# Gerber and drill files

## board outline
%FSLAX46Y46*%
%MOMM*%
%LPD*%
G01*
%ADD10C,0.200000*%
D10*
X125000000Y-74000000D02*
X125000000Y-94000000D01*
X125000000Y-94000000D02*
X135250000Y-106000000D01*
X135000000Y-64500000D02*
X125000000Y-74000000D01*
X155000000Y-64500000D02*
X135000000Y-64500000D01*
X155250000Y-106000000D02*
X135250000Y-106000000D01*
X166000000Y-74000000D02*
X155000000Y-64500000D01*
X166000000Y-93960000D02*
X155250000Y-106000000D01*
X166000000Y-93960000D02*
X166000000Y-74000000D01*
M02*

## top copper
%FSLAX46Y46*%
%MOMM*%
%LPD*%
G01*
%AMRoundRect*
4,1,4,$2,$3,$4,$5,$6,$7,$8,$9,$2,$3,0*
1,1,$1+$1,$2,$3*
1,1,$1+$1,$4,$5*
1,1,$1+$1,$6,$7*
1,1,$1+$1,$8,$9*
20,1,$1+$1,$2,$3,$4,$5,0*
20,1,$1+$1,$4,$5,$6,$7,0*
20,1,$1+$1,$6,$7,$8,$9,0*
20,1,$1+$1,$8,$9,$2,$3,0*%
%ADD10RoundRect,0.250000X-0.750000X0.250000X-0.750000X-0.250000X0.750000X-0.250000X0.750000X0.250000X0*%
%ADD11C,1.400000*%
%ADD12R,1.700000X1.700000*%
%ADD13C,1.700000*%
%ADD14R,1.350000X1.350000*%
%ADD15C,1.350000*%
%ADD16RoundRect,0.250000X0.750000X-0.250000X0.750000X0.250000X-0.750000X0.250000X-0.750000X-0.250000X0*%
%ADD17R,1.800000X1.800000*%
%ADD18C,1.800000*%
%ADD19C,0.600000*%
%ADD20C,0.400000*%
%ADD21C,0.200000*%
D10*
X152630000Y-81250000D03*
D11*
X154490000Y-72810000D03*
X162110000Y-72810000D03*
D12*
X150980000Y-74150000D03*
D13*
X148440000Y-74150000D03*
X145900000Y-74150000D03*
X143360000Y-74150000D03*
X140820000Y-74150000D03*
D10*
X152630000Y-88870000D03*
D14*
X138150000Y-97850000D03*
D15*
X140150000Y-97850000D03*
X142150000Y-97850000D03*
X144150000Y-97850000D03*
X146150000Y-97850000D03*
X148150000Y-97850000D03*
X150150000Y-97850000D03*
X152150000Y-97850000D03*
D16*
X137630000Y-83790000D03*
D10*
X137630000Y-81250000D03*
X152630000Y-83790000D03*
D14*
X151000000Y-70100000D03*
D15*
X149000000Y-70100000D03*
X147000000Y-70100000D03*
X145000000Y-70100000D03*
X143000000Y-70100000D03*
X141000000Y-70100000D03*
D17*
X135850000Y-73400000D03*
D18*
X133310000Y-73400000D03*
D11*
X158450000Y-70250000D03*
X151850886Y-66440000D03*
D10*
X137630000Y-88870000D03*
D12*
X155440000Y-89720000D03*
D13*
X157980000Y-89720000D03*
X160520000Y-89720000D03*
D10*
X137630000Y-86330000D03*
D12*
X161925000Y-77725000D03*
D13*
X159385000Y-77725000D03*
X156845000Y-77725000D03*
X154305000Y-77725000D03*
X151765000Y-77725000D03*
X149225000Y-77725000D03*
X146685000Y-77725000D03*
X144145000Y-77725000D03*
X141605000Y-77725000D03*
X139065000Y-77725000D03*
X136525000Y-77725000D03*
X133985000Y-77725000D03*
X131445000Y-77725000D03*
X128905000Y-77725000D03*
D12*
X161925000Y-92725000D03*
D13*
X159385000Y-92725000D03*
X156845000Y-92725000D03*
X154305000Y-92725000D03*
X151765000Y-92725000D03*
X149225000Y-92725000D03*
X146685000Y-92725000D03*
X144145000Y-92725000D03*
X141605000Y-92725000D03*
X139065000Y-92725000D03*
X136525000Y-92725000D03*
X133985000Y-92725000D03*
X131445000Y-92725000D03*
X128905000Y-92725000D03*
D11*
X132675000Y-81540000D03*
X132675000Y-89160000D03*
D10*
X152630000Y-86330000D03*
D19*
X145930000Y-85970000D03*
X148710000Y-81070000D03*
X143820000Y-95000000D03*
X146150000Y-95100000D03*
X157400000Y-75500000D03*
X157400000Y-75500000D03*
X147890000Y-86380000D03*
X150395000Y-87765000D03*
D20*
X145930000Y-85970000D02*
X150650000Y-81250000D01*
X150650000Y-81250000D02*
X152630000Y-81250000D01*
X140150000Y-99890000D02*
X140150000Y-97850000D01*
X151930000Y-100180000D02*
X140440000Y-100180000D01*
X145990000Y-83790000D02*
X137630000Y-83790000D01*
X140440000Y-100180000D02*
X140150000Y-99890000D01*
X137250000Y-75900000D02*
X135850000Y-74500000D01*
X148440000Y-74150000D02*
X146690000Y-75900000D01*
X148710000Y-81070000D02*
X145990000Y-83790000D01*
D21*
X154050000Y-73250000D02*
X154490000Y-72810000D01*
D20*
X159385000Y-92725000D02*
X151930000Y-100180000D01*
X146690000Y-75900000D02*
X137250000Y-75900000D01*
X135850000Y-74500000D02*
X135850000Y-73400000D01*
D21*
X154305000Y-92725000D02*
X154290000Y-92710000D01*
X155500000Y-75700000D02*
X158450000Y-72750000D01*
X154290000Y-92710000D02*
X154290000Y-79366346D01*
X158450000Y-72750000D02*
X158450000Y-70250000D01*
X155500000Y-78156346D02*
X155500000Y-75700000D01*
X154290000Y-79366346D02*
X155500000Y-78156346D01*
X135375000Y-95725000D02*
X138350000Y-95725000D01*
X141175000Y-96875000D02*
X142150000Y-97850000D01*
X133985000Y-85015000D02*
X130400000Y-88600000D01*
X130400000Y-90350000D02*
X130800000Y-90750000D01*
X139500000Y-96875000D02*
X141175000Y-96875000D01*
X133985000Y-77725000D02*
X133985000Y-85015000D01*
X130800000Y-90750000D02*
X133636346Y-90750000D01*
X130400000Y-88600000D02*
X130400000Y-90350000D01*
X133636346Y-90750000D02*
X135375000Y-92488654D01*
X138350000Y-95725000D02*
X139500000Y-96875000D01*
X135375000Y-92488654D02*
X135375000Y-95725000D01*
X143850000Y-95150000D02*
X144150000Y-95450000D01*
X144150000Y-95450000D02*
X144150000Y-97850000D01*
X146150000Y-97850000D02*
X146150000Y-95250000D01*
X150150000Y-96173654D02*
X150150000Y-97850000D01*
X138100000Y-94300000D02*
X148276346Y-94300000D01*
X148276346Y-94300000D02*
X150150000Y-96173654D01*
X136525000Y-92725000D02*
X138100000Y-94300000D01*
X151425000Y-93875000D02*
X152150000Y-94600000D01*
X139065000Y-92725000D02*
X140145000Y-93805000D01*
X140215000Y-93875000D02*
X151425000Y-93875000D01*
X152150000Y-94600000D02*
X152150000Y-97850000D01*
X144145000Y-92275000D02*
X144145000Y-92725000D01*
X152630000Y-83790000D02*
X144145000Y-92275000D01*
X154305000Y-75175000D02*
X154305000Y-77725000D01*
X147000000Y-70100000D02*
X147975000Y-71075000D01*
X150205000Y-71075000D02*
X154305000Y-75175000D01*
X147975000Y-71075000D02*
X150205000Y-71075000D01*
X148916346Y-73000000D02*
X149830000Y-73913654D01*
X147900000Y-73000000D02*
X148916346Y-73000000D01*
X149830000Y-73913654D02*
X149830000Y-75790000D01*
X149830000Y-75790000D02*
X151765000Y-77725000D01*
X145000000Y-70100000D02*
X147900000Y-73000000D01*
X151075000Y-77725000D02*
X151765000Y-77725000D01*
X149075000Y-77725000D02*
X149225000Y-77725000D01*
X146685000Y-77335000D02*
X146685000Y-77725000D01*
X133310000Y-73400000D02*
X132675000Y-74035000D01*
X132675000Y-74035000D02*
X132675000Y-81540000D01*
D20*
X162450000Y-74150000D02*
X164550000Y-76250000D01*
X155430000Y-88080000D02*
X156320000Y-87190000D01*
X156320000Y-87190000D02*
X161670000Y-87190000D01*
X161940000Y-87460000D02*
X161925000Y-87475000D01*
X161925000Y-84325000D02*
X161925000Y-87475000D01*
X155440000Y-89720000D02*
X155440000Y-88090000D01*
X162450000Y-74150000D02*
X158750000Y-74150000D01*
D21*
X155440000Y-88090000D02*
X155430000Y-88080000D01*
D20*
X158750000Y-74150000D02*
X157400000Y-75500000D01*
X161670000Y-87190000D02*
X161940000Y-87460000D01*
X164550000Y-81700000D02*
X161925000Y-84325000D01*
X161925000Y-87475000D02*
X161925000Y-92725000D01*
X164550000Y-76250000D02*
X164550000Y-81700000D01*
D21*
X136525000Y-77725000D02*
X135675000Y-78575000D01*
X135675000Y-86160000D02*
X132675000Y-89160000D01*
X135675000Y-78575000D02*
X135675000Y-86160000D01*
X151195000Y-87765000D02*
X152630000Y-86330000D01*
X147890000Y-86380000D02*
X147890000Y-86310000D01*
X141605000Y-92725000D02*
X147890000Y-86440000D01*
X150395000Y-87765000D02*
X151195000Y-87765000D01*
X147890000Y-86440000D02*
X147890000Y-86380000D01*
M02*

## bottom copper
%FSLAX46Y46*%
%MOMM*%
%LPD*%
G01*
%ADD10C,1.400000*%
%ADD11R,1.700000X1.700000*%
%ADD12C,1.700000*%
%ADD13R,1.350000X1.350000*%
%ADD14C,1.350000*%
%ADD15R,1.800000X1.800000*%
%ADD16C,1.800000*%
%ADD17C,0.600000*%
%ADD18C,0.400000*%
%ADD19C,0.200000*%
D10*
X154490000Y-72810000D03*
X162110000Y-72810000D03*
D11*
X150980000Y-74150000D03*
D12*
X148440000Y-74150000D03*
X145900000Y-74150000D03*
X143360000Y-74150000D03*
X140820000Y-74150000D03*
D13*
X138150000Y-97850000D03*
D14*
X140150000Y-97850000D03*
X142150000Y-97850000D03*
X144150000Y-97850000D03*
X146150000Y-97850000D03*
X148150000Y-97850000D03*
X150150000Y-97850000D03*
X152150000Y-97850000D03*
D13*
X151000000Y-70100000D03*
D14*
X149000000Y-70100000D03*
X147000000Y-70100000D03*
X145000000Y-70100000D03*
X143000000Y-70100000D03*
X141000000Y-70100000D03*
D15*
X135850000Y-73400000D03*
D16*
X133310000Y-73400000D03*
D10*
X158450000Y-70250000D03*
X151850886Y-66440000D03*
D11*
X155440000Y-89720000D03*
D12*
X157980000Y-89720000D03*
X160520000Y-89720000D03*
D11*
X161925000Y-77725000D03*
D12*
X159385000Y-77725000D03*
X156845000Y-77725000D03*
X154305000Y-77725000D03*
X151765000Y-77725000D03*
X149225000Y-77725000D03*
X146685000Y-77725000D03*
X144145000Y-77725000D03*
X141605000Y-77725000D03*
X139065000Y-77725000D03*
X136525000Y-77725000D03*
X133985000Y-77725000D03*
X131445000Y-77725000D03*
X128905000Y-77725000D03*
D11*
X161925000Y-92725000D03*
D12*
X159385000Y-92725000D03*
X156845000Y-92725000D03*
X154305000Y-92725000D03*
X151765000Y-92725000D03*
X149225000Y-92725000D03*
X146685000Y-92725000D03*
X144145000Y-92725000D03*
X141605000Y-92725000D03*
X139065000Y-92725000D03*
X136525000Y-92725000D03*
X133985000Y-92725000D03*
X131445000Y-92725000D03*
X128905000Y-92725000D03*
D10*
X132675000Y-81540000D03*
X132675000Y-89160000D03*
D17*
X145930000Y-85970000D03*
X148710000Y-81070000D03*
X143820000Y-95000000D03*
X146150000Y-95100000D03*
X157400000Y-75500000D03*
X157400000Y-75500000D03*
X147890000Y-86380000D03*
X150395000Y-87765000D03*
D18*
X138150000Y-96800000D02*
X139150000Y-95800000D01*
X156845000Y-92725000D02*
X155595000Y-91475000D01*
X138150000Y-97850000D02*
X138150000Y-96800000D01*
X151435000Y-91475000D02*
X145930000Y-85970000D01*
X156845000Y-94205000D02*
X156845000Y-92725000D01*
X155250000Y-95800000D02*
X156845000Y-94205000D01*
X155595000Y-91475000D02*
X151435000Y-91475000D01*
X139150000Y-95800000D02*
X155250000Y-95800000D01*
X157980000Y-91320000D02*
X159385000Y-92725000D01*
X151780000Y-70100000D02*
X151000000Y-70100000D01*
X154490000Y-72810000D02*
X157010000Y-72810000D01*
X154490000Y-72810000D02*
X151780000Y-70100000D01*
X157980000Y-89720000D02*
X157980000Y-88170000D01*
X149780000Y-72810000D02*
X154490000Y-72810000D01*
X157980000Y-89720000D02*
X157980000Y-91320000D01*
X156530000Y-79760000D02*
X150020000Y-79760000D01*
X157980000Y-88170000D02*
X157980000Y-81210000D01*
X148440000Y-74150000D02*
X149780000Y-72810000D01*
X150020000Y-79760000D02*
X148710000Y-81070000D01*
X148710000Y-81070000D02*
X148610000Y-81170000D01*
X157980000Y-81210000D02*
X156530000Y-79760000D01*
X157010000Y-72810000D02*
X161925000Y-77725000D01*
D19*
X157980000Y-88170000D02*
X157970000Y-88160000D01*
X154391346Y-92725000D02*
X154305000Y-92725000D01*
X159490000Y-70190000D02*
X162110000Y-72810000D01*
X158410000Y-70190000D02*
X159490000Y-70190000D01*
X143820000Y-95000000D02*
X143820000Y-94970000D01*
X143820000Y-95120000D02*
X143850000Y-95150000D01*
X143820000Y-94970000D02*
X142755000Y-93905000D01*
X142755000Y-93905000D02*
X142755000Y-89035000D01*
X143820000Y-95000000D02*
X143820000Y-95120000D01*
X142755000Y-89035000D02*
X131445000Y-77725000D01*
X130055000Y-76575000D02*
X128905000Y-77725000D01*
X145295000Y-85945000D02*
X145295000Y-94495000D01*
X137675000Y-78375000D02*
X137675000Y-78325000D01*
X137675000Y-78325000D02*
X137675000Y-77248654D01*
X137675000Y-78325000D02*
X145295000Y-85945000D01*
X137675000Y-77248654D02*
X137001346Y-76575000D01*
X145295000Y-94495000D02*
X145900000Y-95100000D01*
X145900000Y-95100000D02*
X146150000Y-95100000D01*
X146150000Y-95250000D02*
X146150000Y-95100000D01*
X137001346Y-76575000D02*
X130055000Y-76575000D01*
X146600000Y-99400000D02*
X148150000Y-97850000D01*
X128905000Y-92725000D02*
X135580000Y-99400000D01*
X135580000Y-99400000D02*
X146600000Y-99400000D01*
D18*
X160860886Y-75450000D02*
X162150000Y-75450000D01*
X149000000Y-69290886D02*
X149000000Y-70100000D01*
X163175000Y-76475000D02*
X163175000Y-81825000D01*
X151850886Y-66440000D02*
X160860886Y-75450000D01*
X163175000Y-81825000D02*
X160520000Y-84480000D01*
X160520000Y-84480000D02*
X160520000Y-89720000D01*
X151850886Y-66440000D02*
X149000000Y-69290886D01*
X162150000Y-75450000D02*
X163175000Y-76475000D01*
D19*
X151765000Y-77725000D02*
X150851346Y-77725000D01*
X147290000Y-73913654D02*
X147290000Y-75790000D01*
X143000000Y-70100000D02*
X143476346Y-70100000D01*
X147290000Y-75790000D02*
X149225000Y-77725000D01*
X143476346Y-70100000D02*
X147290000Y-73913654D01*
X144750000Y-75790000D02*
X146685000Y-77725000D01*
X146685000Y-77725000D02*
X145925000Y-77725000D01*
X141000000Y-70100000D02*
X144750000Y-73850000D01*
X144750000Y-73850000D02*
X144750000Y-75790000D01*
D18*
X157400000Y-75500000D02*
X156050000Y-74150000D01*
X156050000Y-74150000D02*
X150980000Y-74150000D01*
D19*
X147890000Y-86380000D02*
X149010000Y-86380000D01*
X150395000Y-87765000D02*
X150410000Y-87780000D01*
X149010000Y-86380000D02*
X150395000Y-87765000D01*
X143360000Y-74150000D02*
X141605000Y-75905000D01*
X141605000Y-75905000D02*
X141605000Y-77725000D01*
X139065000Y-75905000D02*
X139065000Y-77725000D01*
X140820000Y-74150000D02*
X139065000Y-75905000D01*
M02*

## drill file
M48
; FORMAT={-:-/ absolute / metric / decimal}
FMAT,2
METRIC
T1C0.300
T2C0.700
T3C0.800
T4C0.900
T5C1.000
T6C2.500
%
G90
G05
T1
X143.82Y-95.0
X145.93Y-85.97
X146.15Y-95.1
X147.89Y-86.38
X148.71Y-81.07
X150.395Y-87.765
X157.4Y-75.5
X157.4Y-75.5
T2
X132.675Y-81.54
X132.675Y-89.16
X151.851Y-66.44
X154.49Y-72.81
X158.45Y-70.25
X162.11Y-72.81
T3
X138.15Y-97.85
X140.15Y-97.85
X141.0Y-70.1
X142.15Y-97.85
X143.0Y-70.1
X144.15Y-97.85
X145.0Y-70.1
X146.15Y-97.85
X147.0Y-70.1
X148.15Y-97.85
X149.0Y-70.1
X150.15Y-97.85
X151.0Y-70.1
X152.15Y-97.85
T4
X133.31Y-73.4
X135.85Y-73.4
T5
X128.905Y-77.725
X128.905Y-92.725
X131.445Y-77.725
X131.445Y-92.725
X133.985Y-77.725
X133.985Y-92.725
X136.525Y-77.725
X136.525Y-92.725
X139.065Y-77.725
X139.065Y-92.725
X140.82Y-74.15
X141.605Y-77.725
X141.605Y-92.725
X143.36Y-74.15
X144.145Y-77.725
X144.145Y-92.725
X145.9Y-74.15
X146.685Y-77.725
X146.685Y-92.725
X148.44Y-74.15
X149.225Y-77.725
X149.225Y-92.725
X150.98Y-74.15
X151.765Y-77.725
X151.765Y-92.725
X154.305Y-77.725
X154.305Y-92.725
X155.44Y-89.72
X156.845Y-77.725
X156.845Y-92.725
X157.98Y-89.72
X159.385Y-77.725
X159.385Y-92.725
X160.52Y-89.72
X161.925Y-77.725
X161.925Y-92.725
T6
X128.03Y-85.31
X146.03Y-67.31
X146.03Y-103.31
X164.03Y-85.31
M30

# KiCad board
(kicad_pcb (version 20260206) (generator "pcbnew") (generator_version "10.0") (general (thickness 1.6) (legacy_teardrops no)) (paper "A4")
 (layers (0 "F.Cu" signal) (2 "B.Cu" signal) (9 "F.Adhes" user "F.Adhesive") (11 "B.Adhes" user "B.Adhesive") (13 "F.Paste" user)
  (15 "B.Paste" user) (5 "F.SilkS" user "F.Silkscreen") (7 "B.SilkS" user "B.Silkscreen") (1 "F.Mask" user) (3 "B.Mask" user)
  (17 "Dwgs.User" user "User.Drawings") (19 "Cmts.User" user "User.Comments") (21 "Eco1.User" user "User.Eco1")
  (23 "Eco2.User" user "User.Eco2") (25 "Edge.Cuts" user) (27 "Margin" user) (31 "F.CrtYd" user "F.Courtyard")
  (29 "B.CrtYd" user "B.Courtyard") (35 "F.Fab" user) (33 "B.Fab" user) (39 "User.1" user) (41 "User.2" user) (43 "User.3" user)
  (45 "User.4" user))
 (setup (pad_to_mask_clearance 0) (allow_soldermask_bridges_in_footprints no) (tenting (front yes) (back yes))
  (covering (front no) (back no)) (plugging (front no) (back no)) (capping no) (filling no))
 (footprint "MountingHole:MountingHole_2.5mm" (layer "F.Cu") (at 154.997 70.924)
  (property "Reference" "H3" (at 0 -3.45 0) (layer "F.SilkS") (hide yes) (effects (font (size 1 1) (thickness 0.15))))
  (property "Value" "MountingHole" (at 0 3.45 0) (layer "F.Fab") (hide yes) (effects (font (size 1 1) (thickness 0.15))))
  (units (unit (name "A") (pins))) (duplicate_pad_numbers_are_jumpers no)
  (pad "" np_thru_hole circle (at 9.033 14.386) (size 2.5 2.5) (drill 2.5) (layers "*.Cu" "*.Mask")))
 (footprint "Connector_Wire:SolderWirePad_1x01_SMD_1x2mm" (layer "F.Cu") (at 152.63 81.25 -90)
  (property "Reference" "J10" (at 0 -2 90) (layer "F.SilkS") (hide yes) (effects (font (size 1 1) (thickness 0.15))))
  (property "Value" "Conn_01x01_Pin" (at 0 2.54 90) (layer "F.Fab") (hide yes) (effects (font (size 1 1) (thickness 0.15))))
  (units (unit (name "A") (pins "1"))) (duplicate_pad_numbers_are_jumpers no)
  (pad "1" smd roundrect (at 0 0 270) (size 1 2) (layers "F.Cu" "F.Mask") (roundrect_rratio 0.25) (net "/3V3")))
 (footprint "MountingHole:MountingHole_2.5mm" (layer "F.Cu") (at 126.93 68.71)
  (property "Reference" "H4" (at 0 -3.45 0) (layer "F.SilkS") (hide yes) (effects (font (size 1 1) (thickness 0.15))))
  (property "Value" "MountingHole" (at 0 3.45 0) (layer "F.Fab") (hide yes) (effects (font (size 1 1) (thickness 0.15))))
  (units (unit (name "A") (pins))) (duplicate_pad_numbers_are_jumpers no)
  (pad "" np_thru_hole circle (at 1.1 16.6) (size 2.5 2.5) (drill 2.5) (layers "*.Cu" "*.Mask")))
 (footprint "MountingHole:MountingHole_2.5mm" (layer "F.Cu") (at 147.106 84.455)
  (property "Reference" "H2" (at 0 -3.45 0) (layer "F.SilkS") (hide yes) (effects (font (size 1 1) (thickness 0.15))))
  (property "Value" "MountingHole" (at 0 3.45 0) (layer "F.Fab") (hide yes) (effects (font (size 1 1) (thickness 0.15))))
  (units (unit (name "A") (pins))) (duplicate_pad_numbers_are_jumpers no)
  (pad "" np_thru_hole circle (at -1.076 18.855) (size 2.5 2.5) (drill 2.5) (layers "*.Cu" "*.Mask")))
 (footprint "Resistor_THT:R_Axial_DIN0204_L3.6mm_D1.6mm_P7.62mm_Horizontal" (layer "F.Cu") (at 154.49 72.81)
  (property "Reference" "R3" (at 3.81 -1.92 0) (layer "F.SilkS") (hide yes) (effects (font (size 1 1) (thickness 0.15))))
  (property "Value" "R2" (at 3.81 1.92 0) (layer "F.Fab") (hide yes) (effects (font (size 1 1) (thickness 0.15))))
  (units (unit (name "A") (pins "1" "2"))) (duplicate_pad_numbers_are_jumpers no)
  (pad "1" thru_hole circle (at 0 0) (size 1.4 1.4) (drill 0.7) (layers "*.Cu" "*.Mask") (remove_unused_layers no) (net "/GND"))
  (pad "2" thru_hole circle (at 7.62 0) (size 1.4 1.4) (drill 0.7) (layers "*.Cu" "*.Mask") (remove_unused_layers no) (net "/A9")))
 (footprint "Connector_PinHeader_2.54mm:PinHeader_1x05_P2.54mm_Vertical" (layer "F.Cu") (at 150.98 74.15 -90)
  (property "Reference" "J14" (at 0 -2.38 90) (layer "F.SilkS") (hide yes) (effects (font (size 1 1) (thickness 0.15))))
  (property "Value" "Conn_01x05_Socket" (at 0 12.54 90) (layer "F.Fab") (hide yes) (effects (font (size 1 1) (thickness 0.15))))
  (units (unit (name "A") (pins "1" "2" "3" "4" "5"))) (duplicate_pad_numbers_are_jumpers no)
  (pad "1" thru_hole rect (at 0 0 270) (size 1.7 1.7) (drill 1) (layers "*.Cu" "*.Mask") (remove_unused_layers no) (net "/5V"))
  (pad "2" thru_hole circle (at 0 2.54 270) (size 1.7 1.7) (drill 1) (layers "*.Cu" "*.Mask") (remove_unused_layers no) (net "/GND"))
  (pad "3" thru_hole circle (at 0 5.08 270) (size 1.7 1.7) (drill 1) (layers "*.Cu" "*.Mask") (remove_unused_layers no)
   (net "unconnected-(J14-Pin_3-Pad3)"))
  (pad "4" thru_hole circle (at 0 7.62 270) (size 1.7 1.7) (drill 1) (layers "*.Cu" "*.Mask") (remove_unused_layers no) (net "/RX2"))
  (pad "5" thru_hole circle (at 0 10.16 270) (size 1.7 1.7) (drill 1) (layers "*.Cu" "*.Mask") (remove_unused_layers no) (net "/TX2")))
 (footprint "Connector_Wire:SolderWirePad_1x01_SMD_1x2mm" (layer "F.Cu") (at 152.63 88.87 -90)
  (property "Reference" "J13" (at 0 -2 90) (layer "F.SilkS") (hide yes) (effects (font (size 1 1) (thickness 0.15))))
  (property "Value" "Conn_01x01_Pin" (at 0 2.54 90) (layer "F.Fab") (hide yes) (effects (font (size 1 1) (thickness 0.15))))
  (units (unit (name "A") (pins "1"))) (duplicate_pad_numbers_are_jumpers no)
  (pad "1" smd roundrect (at 0 0 270) (size 1 2) (layers "F.Cu" "F.Mask") (roundrect_rratio 0.25) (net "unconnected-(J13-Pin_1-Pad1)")))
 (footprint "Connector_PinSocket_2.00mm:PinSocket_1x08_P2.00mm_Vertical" (layer "F.Cu") (at 138.15 97.85 90)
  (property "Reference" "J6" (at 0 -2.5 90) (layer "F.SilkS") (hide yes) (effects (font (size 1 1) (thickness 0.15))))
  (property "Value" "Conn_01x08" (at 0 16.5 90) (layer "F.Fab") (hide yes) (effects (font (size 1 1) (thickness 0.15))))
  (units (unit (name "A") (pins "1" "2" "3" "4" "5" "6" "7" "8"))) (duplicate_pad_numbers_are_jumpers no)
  (pad "1" thru_hole rect (at 0 0 90) (size 1.35 1.35) (drill 0.8) (layers "*.Cu" "*.Mask") (remove_unused_layers no) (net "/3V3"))
  (pad "2" thru_hole circle (at 0 2 90) (size 1.35 1.35) (drill 0.8) (layers "*.Cu" "*.Mask") (remove_unused_layers no) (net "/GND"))
  (pad "3" thru_hole circle (at 0 4 90) (size 1.35 1.35) (drill 0.8) (layers "*.Cu" "*.Mask") (remove_unused_layers no) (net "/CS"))
  (pad "4" thru_hole circle (at 0 6 90) (size 1.35 1.35) (drill 0.8) (layers "*.Cu" "*.Mask") (remove_unused_layers no) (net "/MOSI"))
  (pad "5" thru_hole circle (at 0 8 90) (size 1.35 1.35) (drill 0.8) (layers "*.Cu" "*.Mask") (remove_unused_layers no) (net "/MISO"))
  (pad "6" thru_hole circle (at 0 10 90) (size 1.35 1.35) (drill 0.8) (layers "*.Cu" "*.Mask") (remove_unused_layers no) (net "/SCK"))
  (pad "7" thru_hole circle (at 0 12 90) (size 1.35 1.35) (drill 0.8) (layers "*.Cu" "*.Mask") (remove_unused_layers no) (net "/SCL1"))
  (pad "8" thru_hole circle (at 0 14 90) (size 1.35 1.35) (drill 0.8) (layers "*.Cu" "*.Mask") (remove_unused_layers no) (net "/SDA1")))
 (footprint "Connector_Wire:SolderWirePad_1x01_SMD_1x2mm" (layer "F.Cu") (at 137.63 83.79 90)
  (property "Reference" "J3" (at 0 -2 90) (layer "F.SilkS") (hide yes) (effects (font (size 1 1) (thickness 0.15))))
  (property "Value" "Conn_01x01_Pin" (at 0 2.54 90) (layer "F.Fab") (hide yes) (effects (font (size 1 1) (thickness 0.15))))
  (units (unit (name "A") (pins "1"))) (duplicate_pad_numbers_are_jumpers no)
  (pad "1" smd roundrect (at 0 0 90) (size 1 2) (layers "F.Cu" "F.Mask") (roundrect_rratio 0.25) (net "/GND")))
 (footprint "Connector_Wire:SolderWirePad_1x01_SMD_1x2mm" (layer "F.Cu") (at 137.63 81.25 -90)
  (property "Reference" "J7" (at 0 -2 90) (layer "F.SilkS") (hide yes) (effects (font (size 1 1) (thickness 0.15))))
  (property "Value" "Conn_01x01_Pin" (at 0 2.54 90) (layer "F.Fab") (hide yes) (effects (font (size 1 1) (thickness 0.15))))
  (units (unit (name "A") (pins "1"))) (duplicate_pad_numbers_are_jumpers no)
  (pad "1" smd roundrect (at 0 0 270) (size 1 2) (layers "F.Cu" "F.Mask") (roundrect_rratio 0.25) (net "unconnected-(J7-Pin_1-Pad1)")))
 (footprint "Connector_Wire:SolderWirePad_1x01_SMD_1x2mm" (layer "F.Cu") (at 152.63 83.79 -90)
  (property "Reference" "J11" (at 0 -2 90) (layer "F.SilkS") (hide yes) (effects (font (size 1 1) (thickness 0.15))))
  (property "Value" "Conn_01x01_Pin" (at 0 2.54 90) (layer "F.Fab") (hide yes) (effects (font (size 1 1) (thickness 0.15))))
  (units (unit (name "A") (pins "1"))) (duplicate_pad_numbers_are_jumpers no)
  (pad "1" smd roundrect (at 0 0 270) (size 1 2) (layers "F.Cu" "F.Mask") (roundrect_rratio 0.25) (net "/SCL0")))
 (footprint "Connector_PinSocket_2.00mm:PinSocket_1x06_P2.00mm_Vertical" (layer "F.Cu") (at 151 70.1 -90)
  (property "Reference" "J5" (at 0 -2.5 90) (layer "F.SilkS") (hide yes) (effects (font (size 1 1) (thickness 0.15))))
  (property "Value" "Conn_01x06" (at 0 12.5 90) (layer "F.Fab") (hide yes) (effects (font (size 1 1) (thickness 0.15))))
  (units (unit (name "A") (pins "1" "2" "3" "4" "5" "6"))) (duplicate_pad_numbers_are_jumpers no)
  (pad "1" thru_hole rect (at 0 0 270) (size 1.35 1.35) (drill 0.8) (layers "*.Cu" "*.Mask") (remove_unused_layers no) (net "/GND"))
  (pad "2" thru_hole circle (at 0 2 270) (size 1.35 1.35) (drill 0.8) (layers "*.Cu" "*.Mask") (remove_unused_layers no) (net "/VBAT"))
  (pad "3" thru_hole circle (at 0 4 270) (size 1.35 1.35) (drill 0.8) (layers "*.Cu" "*.Mask") (remove_unused_layers no) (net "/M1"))
  (pad "4" thru_hole circle (at 0 6 270) (size 1.35 1.35) (drill 0.8) (layers "*.Cu" "*.Mask") (remove_unused_layers no) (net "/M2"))
  (pad "5" thru_hole circle (at 0 8 270) (size 1.35 1.35) (drill 0.8) (layers "*.Cu" "*.Mask") (remove_unused_layers no) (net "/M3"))
  (pad "6" thru_hole circle (at 0 10 270) (size 1.35 1.35) (drill 0.8) (layers "*.Cu" "*.Mask") (remove_unused_layers no) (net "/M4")))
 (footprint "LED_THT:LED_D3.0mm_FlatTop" (layer "F.Cu") (at 135.85 73.4 180)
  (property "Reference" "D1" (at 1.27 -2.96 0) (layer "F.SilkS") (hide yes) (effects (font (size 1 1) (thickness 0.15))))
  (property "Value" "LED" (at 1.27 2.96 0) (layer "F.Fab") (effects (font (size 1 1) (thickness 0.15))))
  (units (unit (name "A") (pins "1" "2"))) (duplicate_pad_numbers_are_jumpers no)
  (pad "1" thru_hole rect (at 0 0 180) (size 1.8 1.8) (drill 0.9) (layers "*.Cu" "*.Mask") (remove_unused_layers no) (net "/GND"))
  (pad "2" thru_hole circle (at 2.54 0 180) (size 1.8 1.8) (drill 0.9) (layers "*.Cu" "*.Mask") (remove_unused_layers no) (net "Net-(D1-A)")))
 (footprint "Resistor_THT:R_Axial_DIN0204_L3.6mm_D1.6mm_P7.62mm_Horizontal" (layer "F.Cu") (at 158.45 70.25 150)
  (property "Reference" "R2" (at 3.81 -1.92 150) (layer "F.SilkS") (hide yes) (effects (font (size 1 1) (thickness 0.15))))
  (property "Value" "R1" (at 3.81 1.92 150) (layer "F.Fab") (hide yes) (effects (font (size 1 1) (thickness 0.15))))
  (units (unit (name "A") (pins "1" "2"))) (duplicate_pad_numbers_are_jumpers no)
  (pad "1" thru_hole circle (at 0 0 150) (size 1.4 1.4) (drill 0.7) (layers "*.Cu" "*.Mask") (remove_unused_layers no) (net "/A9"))
  (pad "2" thru_hole circle (at 7.62 0 150) (size 1.4 1.4) (drill 0.7) (layers "*.Cu" "*.Mask") (remove_unused_layers no) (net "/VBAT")))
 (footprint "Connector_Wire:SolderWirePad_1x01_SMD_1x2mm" (layer "F.Cu") (at 137.63 88.87 -90)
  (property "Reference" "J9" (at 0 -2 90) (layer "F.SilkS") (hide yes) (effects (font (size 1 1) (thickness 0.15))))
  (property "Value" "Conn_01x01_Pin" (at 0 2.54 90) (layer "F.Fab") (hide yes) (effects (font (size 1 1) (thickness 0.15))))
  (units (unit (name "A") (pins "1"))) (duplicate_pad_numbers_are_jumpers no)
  (pad "1" smd roundrect (at 0 0 270) (size 1 2) (layers "F.Cu" "F.Mask") (roundrect_rratio 0.25) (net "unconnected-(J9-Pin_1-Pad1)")))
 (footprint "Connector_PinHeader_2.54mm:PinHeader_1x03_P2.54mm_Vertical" (layer "F.Cu") (at 155.44 89.72 90)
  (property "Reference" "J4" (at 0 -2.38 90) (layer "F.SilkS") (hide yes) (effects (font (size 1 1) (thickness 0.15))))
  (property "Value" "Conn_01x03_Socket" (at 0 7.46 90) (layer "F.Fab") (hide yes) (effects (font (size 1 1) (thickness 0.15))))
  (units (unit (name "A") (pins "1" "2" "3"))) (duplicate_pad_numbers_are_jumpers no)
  (pad "1" thru_hole rect (at 0 0 90) (size 1.7 1.7) (drill 1) (layers "*.Cu" "*.Mask") (remove_unused_layers no) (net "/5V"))
  (pad "2" thru_hole circle (at 0 2.54 90) (size 1.7 1.7) (drill 1) (layers "*.Cu" "*.Mask") (remove_unused_layers no) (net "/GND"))
  (pad "3" thru_hole circle (at 0 5.08 90) (size 1.7 1.7) (drill 1) (layers "*.Cu" "*.Mask") (remove_unused_layers no) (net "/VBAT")))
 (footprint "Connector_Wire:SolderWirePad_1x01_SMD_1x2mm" (layer "F.Cu") (at 137.63 86.33 -90)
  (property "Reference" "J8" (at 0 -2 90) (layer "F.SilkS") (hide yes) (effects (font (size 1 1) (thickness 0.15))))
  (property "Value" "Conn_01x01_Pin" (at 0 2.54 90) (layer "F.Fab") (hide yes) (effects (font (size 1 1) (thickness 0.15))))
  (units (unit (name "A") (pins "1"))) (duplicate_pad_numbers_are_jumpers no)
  (pad "1" smd roundrect (at 0 0 270) (size 1 2) (layers "F.Cu" "F.Mask") (roundrect_rratio 0.25) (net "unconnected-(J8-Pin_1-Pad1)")))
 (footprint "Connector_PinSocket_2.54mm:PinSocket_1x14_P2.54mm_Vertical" (layer "F.Cu") (at 161.925 77.725 -90)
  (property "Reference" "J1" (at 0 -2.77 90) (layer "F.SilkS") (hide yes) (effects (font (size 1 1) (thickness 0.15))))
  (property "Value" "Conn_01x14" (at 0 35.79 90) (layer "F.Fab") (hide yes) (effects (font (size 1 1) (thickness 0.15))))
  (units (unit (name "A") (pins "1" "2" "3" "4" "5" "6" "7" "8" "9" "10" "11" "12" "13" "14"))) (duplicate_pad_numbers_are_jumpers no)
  (pad "1" thru_hole rect (at 0 0 270) (size 1.7 1.7) (drill 1) (layers "*.Cu" "*.Mask") (remove_unused_layers no) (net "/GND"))
  (pad "2" thru_hole circle (at 0 2.54 270) (size 1.7 1.7) (drill 1) (layers "*.Cu" "*.Mask") (remove_unused_layers no) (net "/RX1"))
  (pad "3" thru_hole circle (at 0 5.08 270) (size 1.7 1.7) (drill 1) (layers "*.Cu" "*.Mask") (remove_unused_layers no) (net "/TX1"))
  (pad "4" thru_hole circle (at 0 7.62 270) (size 1.7 1.7) (drill 1) (layers "*.Cu" "*.Mask") (remove_unused_layers no) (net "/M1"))
  (pad "5" thru_hole circle (at 0 10.16 270) (size 1.7 1.7) (drill 1) (layers "*.Cu" "*.Mask") (remove_unused_layers no) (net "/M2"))
  (pad "6" thru_hole circle (at 0 12.7 270) (size 1.7 1.7) (drill 1) (layers "*.Cu" "*.Mask") (remove_unused_layers no) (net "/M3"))
  (pad "7" thru_hole circle (at 0 15.24 270) (size 1.7 1.7) (drill 1) (layers "*.Cu" "*.Mask") (remove_unused_layers no) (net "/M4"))
  (pad "8" thru_hole circle (at 0 17.78 270) (size 1.7 1.7) (drill 1) (layers "*.Cu" "*.Mask") (remove_unused_layers no)
   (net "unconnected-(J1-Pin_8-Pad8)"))
  (pad "9" thru_hole circle (at 0 20.32 270) (size 1.7 1.7) (drill 1) (layers "*.Cu" "*.Mask") (remove_unused_layers no) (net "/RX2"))
  (pad "10" thru_hole circle (at 0 22.86 270) (size 1.7 1.7) (drill 1) (layers "*.Cu" "*.Mask") (remove_unused_layers no) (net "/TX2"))
  (pad "11" thru_hole circle (at 0 25.4 270) (size 1.7 1.7) (drill 1) (layers "*.Cu" "*.Mask") (remove_unused_layers no) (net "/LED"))
  (pad "12" thru_hole circle (at 0 27.94 270) (size 1.7 1.7) (drill 1) (layers "*.Cu" "*.Mask") (remove_unused_layers no) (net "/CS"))
  (pad "13" thru_hole circle (at 0 30.48 270) (size 1.7 1.7) (drill 1) (layers "*.Cu" "*.Mask") (remove_unused_layers no) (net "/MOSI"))
  (pad "14" thru_hole circle (at 0 33.02 270) (size 1.7 1.7) (drill 1) (layers "*.Cu" "*.Mask") (remove_unused_layers no) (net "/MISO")))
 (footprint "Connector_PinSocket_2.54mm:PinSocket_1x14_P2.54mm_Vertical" (layer "F.Cu") (at 161.925 92.725 -90)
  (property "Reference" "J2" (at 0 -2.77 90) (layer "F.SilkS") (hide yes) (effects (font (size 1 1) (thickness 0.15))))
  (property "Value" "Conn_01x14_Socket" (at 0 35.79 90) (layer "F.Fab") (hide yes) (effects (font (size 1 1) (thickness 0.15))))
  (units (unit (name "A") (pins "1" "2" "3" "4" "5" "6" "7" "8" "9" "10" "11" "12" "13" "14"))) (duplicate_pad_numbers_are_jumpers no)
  (pad "1" thru_hole rect (at 0 0 270) (size 1.7 1.7) (drill 1) (layers "*.Cu" "*.Mask") (remove_unused_layers no) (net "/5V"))
  (pad "2" thru_hole circle (at 0 2.54 270) (size 1.7 1.7) (drill 1) (layers "*.Cu" "*.Mask") (remove_unused_layers no) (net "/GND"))
  (pad "3" thru_hole circle (at 0 5.08 270) (size 1.7 1.7) (drill 1) (layers "*.Cu" "*.Mask") (remove_unused_layers no) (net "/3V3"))
  (pad "4" thru_hole circle (at 0 7.62 270) (size 1.7 1.7) (drill 1) (layers "*.Cu" "*.Mask") (remove_unused_layers no) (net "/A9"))
  (pad "5" thru_hole circle (at 0 10.16 270) (size 1.7 1.7) (drill 1) (layers "*.Cu" "*.Mask") (remove_unused_layers no)
   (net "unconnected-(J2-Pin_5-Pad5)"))
  (pad "6" thru_hole circle (at 0 12.7 270) (size 1.7 1.7) (drill 1) (layers "*.Cu" "*.Mask") (remove_unused_layers no)
   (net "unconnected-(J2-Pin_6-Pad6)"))
  (pad "7" thru_hole circle (at 0 15.24 270) (size 1.7 1.7) (drill 1) (layers "*.Cu" "*.Mask") (remove_unused_layers no)
   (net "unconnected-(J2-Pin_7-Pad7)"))
  (pad "8" thru_hole circle (at 0 17.78 270) (size 1.7 1.7) (drill 1) (layers "*.Cu" "*.Mask") (remove_unused_layers no) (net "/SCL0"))
  (pad "9" thru_hole circle (at 0 20.32 270) (size 1.7 1.7) (drill 1) (layers "*.Cu" "*.Mask") (remove_unused_layers no) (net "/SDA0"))
  (pad "10" thru_hole circle (at 0 22.86 270) (size 1.7 1.7) (drill 1) (layers "*.Cu" "*.Mask") (remove_unused_layers no) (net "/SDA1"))
  (pad "11" thru_hole circle (at 0 25.4 270) (size 1.7 1.7) (drill 1) (layers "*.Cu" "*.Mask") (remove_unused_layers no) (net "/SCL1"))
  (pad "12" thru_hole circle (at 0 27.94 270) (size 1.7 1.7) (drill 1) (layers "*.Cu" "*.Mask") (remove_unused_layers no) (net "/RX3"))
  (pad "13" thru_hole circle (at 0 30.48 270) (size 1.7 1.7) (drill 1) (layers "*.Cu" "*.Mask") (remove_unused_layers no) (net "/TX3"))
  (pad "14" thru_hole circle (at 0 33.02 270) (size 1.7 1.7) (drill 1) (layers "*.Cu" "*.Mask") (remove_unused_layers no) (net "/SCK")))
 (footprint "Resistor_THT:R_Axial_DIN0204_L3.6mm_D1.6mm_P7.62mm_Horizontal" (layer "F.Cu") (at 132.675 82.79 -90)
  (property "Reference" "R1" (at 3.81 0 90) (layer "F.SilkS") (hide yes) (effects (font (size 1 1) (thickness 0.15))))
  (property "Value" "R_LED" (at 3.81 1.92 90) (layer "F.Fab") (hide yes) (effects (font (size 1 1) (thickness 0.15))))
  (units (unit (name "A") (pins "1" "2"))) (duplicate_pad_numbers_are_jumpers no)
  (pad "1" thru_hole circle (at -1.25 0 270) (size 1.4 1.4) (drill 0.7) (layers "*.Cu" "*.Mask") (remove_unused_layers no)
   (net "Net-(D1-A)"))
  (pad "2" thru_hole circle (at 6.37 0 270) (size 1.4 1.4) (drill 0.7) (layers "*.Cu" "*.Mask") (remove_unused_layers no) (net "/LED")))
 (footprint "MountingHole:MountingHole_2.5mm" (layer "F.Cu") (at 143.884038 70.880961 -135)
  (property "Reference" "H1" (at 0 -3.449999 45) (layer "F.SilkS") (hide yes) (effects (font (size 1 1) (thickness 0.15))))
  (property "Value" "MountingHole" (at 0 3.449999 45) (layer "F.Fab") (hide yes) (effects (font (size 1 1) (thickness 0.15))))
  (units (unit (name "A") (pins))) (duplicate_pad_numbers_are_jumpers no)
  (pad "" np_thru_hole circle (at -4.042475 1.007626 225) (size 2.5 2.5) (drill 2.5) (layers "*.Cu" "*.Mask")))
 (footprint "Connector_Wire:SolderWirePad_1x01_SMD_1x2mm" (layer "F.Cu") (at 152.63 86.33 -90)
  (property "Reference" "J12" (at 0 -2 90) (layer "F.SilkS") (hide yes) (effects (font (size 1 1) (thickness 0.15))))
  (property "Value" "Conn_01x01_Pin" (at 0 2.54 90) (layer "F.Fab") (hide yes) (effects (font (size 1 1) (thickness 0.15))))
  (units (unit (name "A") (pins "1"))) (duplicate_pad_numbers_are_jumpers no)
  (pad "1" smd roundrect (at 0 0 270) (size 1 2) (layers "F.Cu" "F.Mask") (roundrect_rratio 0.25) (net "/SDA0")))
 (gr_line (start 125 74) (end 125 94) (stroke (width 0.2) (type solid)) (layer "Edge.Cuts"))
 (gr_line (start 125 94) (end 135.25 106) (stroke (width 0.2) (type solid)) (layer "Edge.Cuts"))
 (gr_line (start 135 64.5) (end 125 74) (stroke (width 0.2) (type solid)) (layer "Edge.Cuts"))
 (gr_line (start 155 64.5) (end 135 64.5) (stroke (width 0.2) (type solid)) (layer "Edge.Cuts"))
 (gr_line (start 155.25 106) (end 135.25 106) (stroke (width 0.2) (type solid)) (layer "Edge.Cuts"))
 (gr_line (start 166 74) (end 155 64.5) (stroke (width 0.2) (type solid)) (layer "Edge.Cuts"))
 (gr_line (start 166 93.96) (end 155.25 106) (stroke (width 0.2) (type solid)) (layer "Edge.Cuts"))
 (gr_line (start 166 93.96) (end 166 74) (stroke (width 0.2) (type solid)) (layer "Edge.Cuts"))
 (segment (start 145.93 85.97) (end 150.65 81.25) (width 0.4) (layer "F.Cu") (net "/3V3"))
 (segment (start 150.65 81.25) (end 152.63 81.25) (width 0.4) (layer "F.Cu") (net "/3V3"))
 (via (at 145.93 85.97) (size 0.6) (drill 0.3) (layers "F.Cu" "B.Cu") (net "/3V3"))
 (segment (start 138.15 96.8) (end 139.15 95.8) (width 0.4) (layer "B.Cu") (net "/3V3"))
 (segment (start 156.845 92.725) (end 155.595 91.475) (width 0.4) (layer "B.Cu") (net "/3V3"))
 (segment (start 138.15 97.85) (end 138.15 96.8) (width 0.4) (layer "B.Cu") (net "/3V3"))
 (segment (start 151.435 91.475) (end 145.93 85.97) (width 0.4) (layer "B.Cu") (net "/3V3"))
 (segment (start 156.845 94.205) (end 156.845 92.725) (width 0.4) (layer "B.Cu") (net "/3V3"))
 (segment (start 155.25 95.8) (end 156.845 94.205) (width 0.4) (layer "B.Cu") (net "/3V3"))
 (segment (start 155.595 91.475) (end 151.435 91.475) (width 0.4) (layer "B.Cu") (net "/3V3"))
 (segment (start 139.15 95.8) (end 155.25 95.8) (width 0.4) (layer "B.Cu") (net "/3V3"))
 (segment (start 140.15 99.89) (end 140.15 97.85) (width 0.4) (layer "F.Cu") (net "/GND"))
 (segment (start 151.93 100.18) (end 140.44 100.18) (width 0.4) (layer "F.Cu") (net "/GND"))
 (segment (start 145.99 83.79) (end 137.63 83.79) (width 0.4) (layer "F.Cu") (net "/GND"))
 (segment (start 140.44 100.18) (end 140.15 99.89) (width 0.4) (layer "F.Cu") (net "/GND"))
 (segment (start 137.25 75.9) (end 135.85 74.5) (width 0.4) (layer "F.Cu") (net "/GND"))
 (segment (start 148.44 74.15) (end 146.69 75.9) (width 0.4) (layer "F.Cu") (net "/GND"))
 (segment (start 148.71 81.07) (end 145.99 83.79) (width 0.4) (layer "F.Cu") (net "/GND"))
 (segment (start 154.05 73.25) (end 154.49 72.81) (width 0.2) (layer "F.Cu") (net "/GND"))
 (segment (start 159.385 92.725) (end 151.93 100.18) (width 0.4) (layer "F.Cu") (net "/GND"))
 (segment (start 146.69 75.9) (end 137.25 75.9) (width 0.4) (layer "F.Cu") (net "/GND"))
 (segment (start 135.85 74.5) (end 135.85 73.4) (width 0.4) (layer "F.Cu") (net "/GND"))
 (via (at 148.71 81.07) (size 0.6) (drill 0.3) (layers "F.Cu" "B.Cu") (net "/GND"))
 (segment (start 157.98 91.32) (end 159.385 92.725) (width 0.4) (layer "B.Cu") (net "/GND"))
 (segment (start 151.78 70.1) (end 151 70.1) (width 0.4) (layer "B.Cu") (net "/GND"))
 (segment (start 154.49 72.81) (end 157.01 72.81) (width 0.4) (layer "B.Cu") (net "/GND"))
 (segment (start 154.49 72.81) (end 151.78 70.1) (width 0.4) (layer "B.Cu") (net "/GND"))
 (segment (start 157.98 89.72) (end 157.98 88.17) (width 0.4) (layer "B.Cu") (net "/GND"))
 (segment (start 149.78 72.81) (end 154.49 72.81) (width 0.4) (layer "B.Cu") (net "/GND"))
 (segment (start 157.98 89.72) (end 157.98 91.32) (width 0.4) (layer "B.Cu") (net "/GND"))
 (segment (start 156.53 79.76) (end 150.02 79.76) (width 0.4) (layer "B.Cu") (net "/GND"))
 (segment (start 157.98 88.17) (end 157.98 81.21) (width 0.4) (layer "B.Cu") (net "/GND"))
 (segment (start 148.44 74.15) (end 149.78 72.81) (width 0.4) (layer "B.Cu") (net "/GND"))
 (segment (start 150.02 79.76) (end 148.71 81.07) (width 0.4) (layer "B.Cu") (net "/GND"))
 (segment (start 148.71 81.07) (end 148.61 81.17) (width 0.4) (layer "B.Cu") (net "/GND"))
 (segment (start 157.98 81.21) (end 156.53 79.76) (width 0.4) (layer "B.Cu") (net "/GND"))
 (segment (start 157.01 72.81) (end 161.925 77.725) (width 0.4) (layer "B.Cu") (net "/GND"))
 (segment (start 157.98 88.17) (end 157.97 88.16) (width 0.2) (layer "B.Cu") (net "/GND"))
 (segment (start 154.305 92.725) (end 154.29 92.71) (width 0.2) (layer "F.Cu") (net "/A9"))
 (segment (start 155.5 75.7) (end 158.45 72.75) (width 0.2) (layer "F.Cu") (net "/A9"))
 (segment (start 154.29 92.71) (end 154.29 79.366346) (width 0.2) (layer "F.Cu") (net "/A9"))
 (segment (start 158.45 72.75) (end 158.45 70.25) (width 0.2) (layer "F.Cu") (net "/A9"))
 (segment (start 155.5 78.156346) (end 155.5 75.7) (width 0.2) (layer "F.Cu") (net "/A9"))
 (segment (start 154.29 79.366346) (end 155.5 78.156346) (width 0.2) (layer "F.Cu") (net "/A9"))
 (segment (start 154.391346 92.725) (end 154.305 92.725) (width 0.2) (layer "B.Cu") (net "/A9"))
 (segment (start 159.49 70.19) (end 162.11 72.81) (width 0.2) (layer "B.Cu") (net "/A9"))
 (segment (start 158.41 70.19) (end 159.49 70.19) (width 0.2) (layer "B.Cu") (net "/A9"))
 (segment (start 135.375 95.725) (end 138.35 95.725) (width 0.2) (layer "F.Cu") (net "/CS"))
 (segment (start 141.175 96.875) (end 142.15 97.85) (width 0.2) (layer "F.Cu") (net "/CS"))
 (segment (start 133.985 85.015) (end 130.4 88.6) (width 0.2) (layer "F.Cu") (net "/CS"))
 (segment (start 130.4 90.35) (end 130.8 90.75) (width 0.2) (layer "F.Cu") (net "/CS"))
 (segment (start 139.5 96.875) (end 141.175 96.875) (width 0.2) (layer "F.Cu") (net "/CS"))
 (segment (start 133.985 77.725) (end 133.985 85.015) (width 0.2) (layer "F.Cu") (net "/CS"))
 (segment (start 130.8 90.75) (end 133.636346 90.75) (width 0.2) (layer "F.Cu") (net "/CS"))
 (segment (start 130.4 88.6) (end 130.4 90.35) (width 0.2) (layer "F.Cu") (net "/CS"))
 (segment (start 133.636346 90.75) (end 135.375 92.488654) (width 0.2) (layer "F.Cu") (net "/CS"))
 (segment (start 138.35 95.725) (end 139.5 96.875) (width 0.2) (layer "F.Cu") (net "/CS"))
 (segment (start 135.375 92.488654) (end 135.375 95.725) (width 0.2) (layer "F.Cu") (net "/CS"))
 (segment (start 143.85 95.15) (end 144.15 95.45) (width 0.2) (layer "F.Cu") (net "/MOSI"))
 (segment (start 144.15 95.45) (end 144.15 97.85) (width 0.2) (layer "F.Cu") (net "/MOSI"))
 (via (at 143.82 95) (size 0.6) (drill 0.3) (layers "F.Cu" "B.Cu") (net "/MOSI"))
 (segment (start 143.82 95) (end 143.82 94.97) (width 0.2) (layer "B.Cu") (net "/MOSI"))
 (segment (start 143.82 95.12) (end 143.85 95.15) (width 0.2) (layer "B.Cu") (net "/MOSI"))
 (segment (start 143.82 94.97) (end 142.755 93.905) (width 0.2) (layer "B.Cu") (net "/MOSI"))
 (segment (start 142.755 93.905) (end 142.755 89.035) (width 0.2) (layer "B.Cu") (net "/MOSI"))
 (segment (start 143.82 95) (end 143.82 95.12) (width 0.2) (layer "B.Cu") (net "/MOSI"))
 (segment (start 142.755 89.035) (end 131.445 77.725) (width 0.2) (layer "B.Cu") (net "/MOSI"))
 (segment (start 146.15 97.85) (end 146.15 95.25) (width 0.2) (layer "F.Cu") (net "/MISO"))
 (via (at 146.15 95.1) (size 0.6) (drill 0.3) (layers "F.Cu" "B.Cu") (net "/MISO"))
 (segment (start 130.055 76.575) (end 128.905 77.725) (width 0.2) (layer "B.Cu") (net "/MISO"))
 (segment (start 145.295 85.945) (end 145.295 94.495) (width 0.2) (layer "B.Cu") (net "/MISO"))
 (segment (start 137.675 78.375) (end 137.675 78.325) (width 0.2) (layer "B.Cu") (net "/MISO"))
 (segment (start 137.675 78.325) (end 137.675 77.248654) (width 0.2) (layer "B.Cu") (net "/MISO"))
 (segment (start 137.675 78.325) (end 145.295 85.945) (width 0.2) (layer "B.Cu") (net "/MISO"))
 (segment (start 137.675 77.248654) (end 137.001346 76.575) (width 0.2) (layer "B.Cu") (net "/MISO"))
 (segment (start 145.295 94.495) (end 145.9 95.1) (width 0.2) (layer "B.Cu") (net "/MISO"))
 (segment (start 145.9 95.1) (end 146.15 95.1) (width 0.2) (layer "B.Cu") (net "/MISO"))
 (segment (start 146.15 95.25) (end 146.15 95.1) (width 0.2) (layer "B.Cu") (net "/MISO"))
 (segment (start 137.001346 76.575) (end 130.055 76.575) (width 0.2) (layer "B.Cu") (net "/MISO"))
 (segment (start 146.6 99.4) (end 148.15 97.85) (width 0.2) (layer "B.Cu") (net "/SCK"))
 (segment (start 128.905 92.725) (end 135.58 99.4) (width 0.2) (layer "B.Cu") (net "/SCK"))
 (segment (start 135.58 99.4) (end 146.6 99.4) (width 0.2) (layer "B.Cu") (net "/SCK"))
 (segment (start 150.15 96.173654) (end 150.15 97.85) (width 0.2) (layer "F.Cu") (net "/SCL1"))
 (segment (start 138.1 94.3) (end 148.276346 94.3) (width 0.2) (layer "F.Cu") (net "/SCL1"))
 (segment (start 148.276346 94.3) (end 150.15 96.173654) (width 0.2) (layer "F.Cu") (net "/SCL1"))
 (segment (start 136.525 92.725) (end 138.1 94.3) (width 0.2) (layer "F.Cu") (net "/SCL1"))
 (segment (start 151.425 93.875) (end 152.15 94.6) (width 0.2) (layer "F.Cu") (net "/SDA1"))
 (segment (start 139.065 92.725) (end 140.145 93.805) (width 0.2) (layer "F.Cu") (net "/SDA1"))
 (segment (start 140.215 93.875) (end 151.425 93.875) (width 0.2) (layer "F.Cu") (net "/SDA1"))
 (segment (start 152.15 94.6) (end 152.15 97.85) (width 0.2) (layer "F.Cu") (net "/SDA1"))
 (segment (start 144.145 92.275) (end 144.145 92.725) (width 0.2) (layer "F.Cu") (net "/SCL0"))
 (segment (start 152.63 83.79) (end 144.145 92.275) (width 0.2) (layer "F.Cu") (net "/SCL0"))
 (segment (start 160.860886 75.45) (end 162.15 75.45) (width 0.4) (layer "B.Cu") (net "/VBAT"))
 (segment (start 149 69.290886) (end 149 70.1) (width 0.4) (layer "B.Cu") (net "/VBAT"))
 (segment (start 163.175 76.475) (end 163.175 81.825) (width 0.4) (layer "B.Cu") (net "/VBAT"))
 (segment (start 151.850886 66.44) (end 160.860886 75.45) (width 0.4) (layer "B.Cu") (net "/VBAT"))
 (segment (start 163.175 81.825) (end 160.52 84.48) (width 0.4) (layer "B.Cu") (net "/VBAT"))
 (segment (start 160.52 84.48) (end 160.52 89.72) (width 0.4) (layer "B.Cu") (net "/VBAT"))
 (segment (start 151.850886 66.44) (end 149 69.290886) (width 0.4) (layer "B.Cu") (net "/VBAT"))
 (segment (start 162.15 75.45) (end 163.175 76.475) (width 0.4) (layer "B.Cu") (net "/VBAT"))
 (segment (start 154.305 75.175) (end 154.305 77.725) (width 0.2) (layer "F.Cu") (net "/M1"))
 (segment (start 147 70.1) (end 147.975 71.075) (width 0.2) (layer "F.Cu") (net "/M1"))
 (segment (start 150.205 71.075) (end 154.305 75.175) (width 0.2) (layer "F.Cu") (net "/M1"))
 (segment (start 147.975 71.075) (end 150.205 71.075) (width 0.2) (layer "F.Cu") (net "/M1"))
 (segment (start 148.916346 73) (end 149.83 73.913654) (width 0.2) (layer "F.Cu") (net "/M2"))
 (segment (start 147.9 73) (end 148.916346 73) (width 0.2) (layer "F.Cu") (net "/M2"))
 (segment (start 149.83 73.913654) (end 149.83 75.79) (width 0.2) (layer "F.Cu") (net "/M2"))
 (segment (start 149.83 75.79) (end 151.765 77.725) (width 0.2) (layer "F.Cu") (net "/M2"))
 (segment (start 145 70.1) (end 147.9 73) (width 0.2) (layer "F.Cu") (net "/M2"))
 (segment (start 151.075 77.725) (end 151.765 77.725) (width 0.2) (layer "F.Cu") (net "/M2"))
 (segment (start 151.765 77.725) (end 150.851346 77.725) (width 0.2) (layer "B.Cu") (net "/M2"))
 (segment (start 149.075 77.725) (end 149.225 77.725) (width 0.2) (layer "F.Cu") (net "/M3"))
 (segment (start 147.29 73.913654) (end 147.29 75.79) (width 0.2) (layer "B.Cu") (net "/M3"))
 (segment (start 143 70.1) (end 143.476346 70.1) (width 0.2) (layer "B.Cu") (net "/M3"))
 (segment (start 147.29 75.79) (end 149.225 77.725) (width 0.2) (layer "B.Cu") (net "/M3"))
 (segment (start 143.476346 70.1) (end 147.29 73.913654) (width 0.2) (layer "B.Cu") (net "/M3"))
 (segment (start 146.685 77.335) (end 146.685 77.725) (width 0.2) (layer "F.Cu") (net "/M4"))
 (segment (start 144.75 75.79) (end 146.685 77.725) (width 0.2) (layer "B.Cu") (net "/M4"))
 (segment (start 146.685 77.725) (end 145.925 77.725) (width 0.2) (layer "B.Cu") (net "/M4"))
 (segment (start 141 70.1) (end 144.75 73.85) (width 0.2) (layer "B.Cu") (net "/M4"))
 (segment (start 144.75 73.85) (end 144.75 75.79) (width 0.2) (layer "B.Cu") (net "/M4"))
 (segment (start 133.31 73.4) (end 132.675 74.035) (width 0.2) (layer "F.Cu") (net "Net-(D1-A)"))
 (segment (start 132.675 74.035) (end 132.675 81.54) (width 0.2) (layer "F.Cu") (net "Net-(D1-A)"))
 (segment (start 162.45 74.15) (end 164.55 76.25) (width 0.4) (layer "F.Cu") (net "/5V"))
 (segment (start 155.43 88.08) (end 156.32 87.19) (width 0.4) (layer "F.Cu") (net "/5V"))
 (segment (start 156.32 87.19) (end 161.67 87.19) (width 0.4) (layer "F.Cu") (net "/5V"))
 (segment (start 161.94 87.46) (end 161.925 87.475) (width 0.4) (layer "F.Cu") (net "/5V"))
 (segment (start 161.925 84.325) (end 161.925 87.475) (width 0.4) (layer "F.Cu") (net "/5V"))
 (segment (start 155.44 89.72) (end 155.44 88.09) (width 0.4) (layer "F.Cu") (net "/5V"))
 (segment (start 162.45 74.15) (end 158.75 74.15) (width 0.4) (layer "F.Cu") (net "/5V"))
 (segment (start 155.44 88.09) (end 155.43 88.08) (width 0.2) (layer "F.Cu") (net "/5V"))
 (segment (start 158.75 74.15) (end 157.4 75.5) (width 0.4) (layer "F.Cu") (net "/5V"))
 (segment (start 161.67 87.19) (end 161.94 87.46) (width 0.4) (layer "F.Cu") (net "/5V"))
 (segment (start 164.55 81.7) (end 161.925 84.325) (width 0.4) (layer "F.Cu") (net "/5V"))
 (segment (start 161.925 87.475) (end 161.925 92.725) (width 0.4) (layer "F.Cu") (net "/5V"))
 (segment (start 164.55 76.25) (end 164.55 81.7) (width 0.4) (layer "F.Cu") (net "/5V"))
 (via (at 157.4 75.5) (size 0.6) (drill 0.3) (layers "F.Cu" "B.Cu") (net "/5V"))
 (via (at 157.4 75.5) (size 0.6) (drill 0.3) (layers "F.Cu" "B.Cu") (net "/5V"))
 (segment (start 157.4 75.5) (end 156.05 74.15) (width 0.4) (layer "B.Cu") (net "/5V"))
 (segment (start 156.05 74.15) (end 150.98 74.15) (width 0.4) (layer "B.Cu") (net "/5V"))
 (segment (start 136.525 77.725) (end 135.675 78.575) (width 0.2) (layer "F.Cu") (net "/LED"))
 (segment (start 135.675 86.16) (end 132.675 89.16) (width 0.2) (layer "F.Cu") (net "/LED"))
 (segment (start 135.675 78.575) (end 135.675 86.16) (width 0.2) (layer "F.Cu") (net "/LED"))
 (segment (start 151.195 87.765) (end 152.63 86.33) (width 0.2) (layer "F.Cu") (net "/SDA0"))
 (segment (start 147.89 86.38) (end 147.89 86.31) (width 0.2) (layer "F.Cu") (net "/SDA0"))
 (segment (start 141.605 92.725) (end 147.89 86.44) (width 0.2) (layer "F.Cu") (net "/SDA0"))
 (segment (start 150.395 87.765) (end 151.195 87.765) (width 0.2) (layer "F.Cu") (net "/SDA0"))
 (segment (start 147.89 86.44) (end 147.89 86.38) (width 0.2) (layer "F.Cu") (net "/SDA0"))
 (via (at 147.89 86.38) (size 0.6) (drill 0.3) (layers "F.Cu" "B.Cu") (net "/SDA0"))
 (via (at 150.395 87.765) (size 0.6) (drill 0.3) (layers "F.Cu" "B.Cu") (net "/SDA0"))
 (segment (start 147.89 86.38) (end 149.01 86.38) (width 0.2) (layer "B.Cu") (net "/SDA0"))
 (segment (start 150.395 87.765) (end 150.41 87.78) (width 0.2) (layer "B.Cu") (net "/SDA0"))
 (segment (start 149.01 86.38) (end 150.395 87.765) (width 0.2) (layer "B.Cu") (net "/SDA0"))
 (segment (start 143.36 74.15) (end 141.605 75.905) (width 0.2) (layer "B.Cu") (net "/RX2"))
 (segment (start 141.605 75.905) (end 141.605 77.725) (width 0.2) (layer "B.Cu") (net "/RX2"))
 (segment (start 139.065 75.905) (end 139.065 77.725) (width 0.2) (layer "B.Cu") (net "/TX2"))
 (segment (start 140.82 74.15) (end 139.065 75.905) (width 0.2) (layer "B.Cu") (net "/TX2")))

